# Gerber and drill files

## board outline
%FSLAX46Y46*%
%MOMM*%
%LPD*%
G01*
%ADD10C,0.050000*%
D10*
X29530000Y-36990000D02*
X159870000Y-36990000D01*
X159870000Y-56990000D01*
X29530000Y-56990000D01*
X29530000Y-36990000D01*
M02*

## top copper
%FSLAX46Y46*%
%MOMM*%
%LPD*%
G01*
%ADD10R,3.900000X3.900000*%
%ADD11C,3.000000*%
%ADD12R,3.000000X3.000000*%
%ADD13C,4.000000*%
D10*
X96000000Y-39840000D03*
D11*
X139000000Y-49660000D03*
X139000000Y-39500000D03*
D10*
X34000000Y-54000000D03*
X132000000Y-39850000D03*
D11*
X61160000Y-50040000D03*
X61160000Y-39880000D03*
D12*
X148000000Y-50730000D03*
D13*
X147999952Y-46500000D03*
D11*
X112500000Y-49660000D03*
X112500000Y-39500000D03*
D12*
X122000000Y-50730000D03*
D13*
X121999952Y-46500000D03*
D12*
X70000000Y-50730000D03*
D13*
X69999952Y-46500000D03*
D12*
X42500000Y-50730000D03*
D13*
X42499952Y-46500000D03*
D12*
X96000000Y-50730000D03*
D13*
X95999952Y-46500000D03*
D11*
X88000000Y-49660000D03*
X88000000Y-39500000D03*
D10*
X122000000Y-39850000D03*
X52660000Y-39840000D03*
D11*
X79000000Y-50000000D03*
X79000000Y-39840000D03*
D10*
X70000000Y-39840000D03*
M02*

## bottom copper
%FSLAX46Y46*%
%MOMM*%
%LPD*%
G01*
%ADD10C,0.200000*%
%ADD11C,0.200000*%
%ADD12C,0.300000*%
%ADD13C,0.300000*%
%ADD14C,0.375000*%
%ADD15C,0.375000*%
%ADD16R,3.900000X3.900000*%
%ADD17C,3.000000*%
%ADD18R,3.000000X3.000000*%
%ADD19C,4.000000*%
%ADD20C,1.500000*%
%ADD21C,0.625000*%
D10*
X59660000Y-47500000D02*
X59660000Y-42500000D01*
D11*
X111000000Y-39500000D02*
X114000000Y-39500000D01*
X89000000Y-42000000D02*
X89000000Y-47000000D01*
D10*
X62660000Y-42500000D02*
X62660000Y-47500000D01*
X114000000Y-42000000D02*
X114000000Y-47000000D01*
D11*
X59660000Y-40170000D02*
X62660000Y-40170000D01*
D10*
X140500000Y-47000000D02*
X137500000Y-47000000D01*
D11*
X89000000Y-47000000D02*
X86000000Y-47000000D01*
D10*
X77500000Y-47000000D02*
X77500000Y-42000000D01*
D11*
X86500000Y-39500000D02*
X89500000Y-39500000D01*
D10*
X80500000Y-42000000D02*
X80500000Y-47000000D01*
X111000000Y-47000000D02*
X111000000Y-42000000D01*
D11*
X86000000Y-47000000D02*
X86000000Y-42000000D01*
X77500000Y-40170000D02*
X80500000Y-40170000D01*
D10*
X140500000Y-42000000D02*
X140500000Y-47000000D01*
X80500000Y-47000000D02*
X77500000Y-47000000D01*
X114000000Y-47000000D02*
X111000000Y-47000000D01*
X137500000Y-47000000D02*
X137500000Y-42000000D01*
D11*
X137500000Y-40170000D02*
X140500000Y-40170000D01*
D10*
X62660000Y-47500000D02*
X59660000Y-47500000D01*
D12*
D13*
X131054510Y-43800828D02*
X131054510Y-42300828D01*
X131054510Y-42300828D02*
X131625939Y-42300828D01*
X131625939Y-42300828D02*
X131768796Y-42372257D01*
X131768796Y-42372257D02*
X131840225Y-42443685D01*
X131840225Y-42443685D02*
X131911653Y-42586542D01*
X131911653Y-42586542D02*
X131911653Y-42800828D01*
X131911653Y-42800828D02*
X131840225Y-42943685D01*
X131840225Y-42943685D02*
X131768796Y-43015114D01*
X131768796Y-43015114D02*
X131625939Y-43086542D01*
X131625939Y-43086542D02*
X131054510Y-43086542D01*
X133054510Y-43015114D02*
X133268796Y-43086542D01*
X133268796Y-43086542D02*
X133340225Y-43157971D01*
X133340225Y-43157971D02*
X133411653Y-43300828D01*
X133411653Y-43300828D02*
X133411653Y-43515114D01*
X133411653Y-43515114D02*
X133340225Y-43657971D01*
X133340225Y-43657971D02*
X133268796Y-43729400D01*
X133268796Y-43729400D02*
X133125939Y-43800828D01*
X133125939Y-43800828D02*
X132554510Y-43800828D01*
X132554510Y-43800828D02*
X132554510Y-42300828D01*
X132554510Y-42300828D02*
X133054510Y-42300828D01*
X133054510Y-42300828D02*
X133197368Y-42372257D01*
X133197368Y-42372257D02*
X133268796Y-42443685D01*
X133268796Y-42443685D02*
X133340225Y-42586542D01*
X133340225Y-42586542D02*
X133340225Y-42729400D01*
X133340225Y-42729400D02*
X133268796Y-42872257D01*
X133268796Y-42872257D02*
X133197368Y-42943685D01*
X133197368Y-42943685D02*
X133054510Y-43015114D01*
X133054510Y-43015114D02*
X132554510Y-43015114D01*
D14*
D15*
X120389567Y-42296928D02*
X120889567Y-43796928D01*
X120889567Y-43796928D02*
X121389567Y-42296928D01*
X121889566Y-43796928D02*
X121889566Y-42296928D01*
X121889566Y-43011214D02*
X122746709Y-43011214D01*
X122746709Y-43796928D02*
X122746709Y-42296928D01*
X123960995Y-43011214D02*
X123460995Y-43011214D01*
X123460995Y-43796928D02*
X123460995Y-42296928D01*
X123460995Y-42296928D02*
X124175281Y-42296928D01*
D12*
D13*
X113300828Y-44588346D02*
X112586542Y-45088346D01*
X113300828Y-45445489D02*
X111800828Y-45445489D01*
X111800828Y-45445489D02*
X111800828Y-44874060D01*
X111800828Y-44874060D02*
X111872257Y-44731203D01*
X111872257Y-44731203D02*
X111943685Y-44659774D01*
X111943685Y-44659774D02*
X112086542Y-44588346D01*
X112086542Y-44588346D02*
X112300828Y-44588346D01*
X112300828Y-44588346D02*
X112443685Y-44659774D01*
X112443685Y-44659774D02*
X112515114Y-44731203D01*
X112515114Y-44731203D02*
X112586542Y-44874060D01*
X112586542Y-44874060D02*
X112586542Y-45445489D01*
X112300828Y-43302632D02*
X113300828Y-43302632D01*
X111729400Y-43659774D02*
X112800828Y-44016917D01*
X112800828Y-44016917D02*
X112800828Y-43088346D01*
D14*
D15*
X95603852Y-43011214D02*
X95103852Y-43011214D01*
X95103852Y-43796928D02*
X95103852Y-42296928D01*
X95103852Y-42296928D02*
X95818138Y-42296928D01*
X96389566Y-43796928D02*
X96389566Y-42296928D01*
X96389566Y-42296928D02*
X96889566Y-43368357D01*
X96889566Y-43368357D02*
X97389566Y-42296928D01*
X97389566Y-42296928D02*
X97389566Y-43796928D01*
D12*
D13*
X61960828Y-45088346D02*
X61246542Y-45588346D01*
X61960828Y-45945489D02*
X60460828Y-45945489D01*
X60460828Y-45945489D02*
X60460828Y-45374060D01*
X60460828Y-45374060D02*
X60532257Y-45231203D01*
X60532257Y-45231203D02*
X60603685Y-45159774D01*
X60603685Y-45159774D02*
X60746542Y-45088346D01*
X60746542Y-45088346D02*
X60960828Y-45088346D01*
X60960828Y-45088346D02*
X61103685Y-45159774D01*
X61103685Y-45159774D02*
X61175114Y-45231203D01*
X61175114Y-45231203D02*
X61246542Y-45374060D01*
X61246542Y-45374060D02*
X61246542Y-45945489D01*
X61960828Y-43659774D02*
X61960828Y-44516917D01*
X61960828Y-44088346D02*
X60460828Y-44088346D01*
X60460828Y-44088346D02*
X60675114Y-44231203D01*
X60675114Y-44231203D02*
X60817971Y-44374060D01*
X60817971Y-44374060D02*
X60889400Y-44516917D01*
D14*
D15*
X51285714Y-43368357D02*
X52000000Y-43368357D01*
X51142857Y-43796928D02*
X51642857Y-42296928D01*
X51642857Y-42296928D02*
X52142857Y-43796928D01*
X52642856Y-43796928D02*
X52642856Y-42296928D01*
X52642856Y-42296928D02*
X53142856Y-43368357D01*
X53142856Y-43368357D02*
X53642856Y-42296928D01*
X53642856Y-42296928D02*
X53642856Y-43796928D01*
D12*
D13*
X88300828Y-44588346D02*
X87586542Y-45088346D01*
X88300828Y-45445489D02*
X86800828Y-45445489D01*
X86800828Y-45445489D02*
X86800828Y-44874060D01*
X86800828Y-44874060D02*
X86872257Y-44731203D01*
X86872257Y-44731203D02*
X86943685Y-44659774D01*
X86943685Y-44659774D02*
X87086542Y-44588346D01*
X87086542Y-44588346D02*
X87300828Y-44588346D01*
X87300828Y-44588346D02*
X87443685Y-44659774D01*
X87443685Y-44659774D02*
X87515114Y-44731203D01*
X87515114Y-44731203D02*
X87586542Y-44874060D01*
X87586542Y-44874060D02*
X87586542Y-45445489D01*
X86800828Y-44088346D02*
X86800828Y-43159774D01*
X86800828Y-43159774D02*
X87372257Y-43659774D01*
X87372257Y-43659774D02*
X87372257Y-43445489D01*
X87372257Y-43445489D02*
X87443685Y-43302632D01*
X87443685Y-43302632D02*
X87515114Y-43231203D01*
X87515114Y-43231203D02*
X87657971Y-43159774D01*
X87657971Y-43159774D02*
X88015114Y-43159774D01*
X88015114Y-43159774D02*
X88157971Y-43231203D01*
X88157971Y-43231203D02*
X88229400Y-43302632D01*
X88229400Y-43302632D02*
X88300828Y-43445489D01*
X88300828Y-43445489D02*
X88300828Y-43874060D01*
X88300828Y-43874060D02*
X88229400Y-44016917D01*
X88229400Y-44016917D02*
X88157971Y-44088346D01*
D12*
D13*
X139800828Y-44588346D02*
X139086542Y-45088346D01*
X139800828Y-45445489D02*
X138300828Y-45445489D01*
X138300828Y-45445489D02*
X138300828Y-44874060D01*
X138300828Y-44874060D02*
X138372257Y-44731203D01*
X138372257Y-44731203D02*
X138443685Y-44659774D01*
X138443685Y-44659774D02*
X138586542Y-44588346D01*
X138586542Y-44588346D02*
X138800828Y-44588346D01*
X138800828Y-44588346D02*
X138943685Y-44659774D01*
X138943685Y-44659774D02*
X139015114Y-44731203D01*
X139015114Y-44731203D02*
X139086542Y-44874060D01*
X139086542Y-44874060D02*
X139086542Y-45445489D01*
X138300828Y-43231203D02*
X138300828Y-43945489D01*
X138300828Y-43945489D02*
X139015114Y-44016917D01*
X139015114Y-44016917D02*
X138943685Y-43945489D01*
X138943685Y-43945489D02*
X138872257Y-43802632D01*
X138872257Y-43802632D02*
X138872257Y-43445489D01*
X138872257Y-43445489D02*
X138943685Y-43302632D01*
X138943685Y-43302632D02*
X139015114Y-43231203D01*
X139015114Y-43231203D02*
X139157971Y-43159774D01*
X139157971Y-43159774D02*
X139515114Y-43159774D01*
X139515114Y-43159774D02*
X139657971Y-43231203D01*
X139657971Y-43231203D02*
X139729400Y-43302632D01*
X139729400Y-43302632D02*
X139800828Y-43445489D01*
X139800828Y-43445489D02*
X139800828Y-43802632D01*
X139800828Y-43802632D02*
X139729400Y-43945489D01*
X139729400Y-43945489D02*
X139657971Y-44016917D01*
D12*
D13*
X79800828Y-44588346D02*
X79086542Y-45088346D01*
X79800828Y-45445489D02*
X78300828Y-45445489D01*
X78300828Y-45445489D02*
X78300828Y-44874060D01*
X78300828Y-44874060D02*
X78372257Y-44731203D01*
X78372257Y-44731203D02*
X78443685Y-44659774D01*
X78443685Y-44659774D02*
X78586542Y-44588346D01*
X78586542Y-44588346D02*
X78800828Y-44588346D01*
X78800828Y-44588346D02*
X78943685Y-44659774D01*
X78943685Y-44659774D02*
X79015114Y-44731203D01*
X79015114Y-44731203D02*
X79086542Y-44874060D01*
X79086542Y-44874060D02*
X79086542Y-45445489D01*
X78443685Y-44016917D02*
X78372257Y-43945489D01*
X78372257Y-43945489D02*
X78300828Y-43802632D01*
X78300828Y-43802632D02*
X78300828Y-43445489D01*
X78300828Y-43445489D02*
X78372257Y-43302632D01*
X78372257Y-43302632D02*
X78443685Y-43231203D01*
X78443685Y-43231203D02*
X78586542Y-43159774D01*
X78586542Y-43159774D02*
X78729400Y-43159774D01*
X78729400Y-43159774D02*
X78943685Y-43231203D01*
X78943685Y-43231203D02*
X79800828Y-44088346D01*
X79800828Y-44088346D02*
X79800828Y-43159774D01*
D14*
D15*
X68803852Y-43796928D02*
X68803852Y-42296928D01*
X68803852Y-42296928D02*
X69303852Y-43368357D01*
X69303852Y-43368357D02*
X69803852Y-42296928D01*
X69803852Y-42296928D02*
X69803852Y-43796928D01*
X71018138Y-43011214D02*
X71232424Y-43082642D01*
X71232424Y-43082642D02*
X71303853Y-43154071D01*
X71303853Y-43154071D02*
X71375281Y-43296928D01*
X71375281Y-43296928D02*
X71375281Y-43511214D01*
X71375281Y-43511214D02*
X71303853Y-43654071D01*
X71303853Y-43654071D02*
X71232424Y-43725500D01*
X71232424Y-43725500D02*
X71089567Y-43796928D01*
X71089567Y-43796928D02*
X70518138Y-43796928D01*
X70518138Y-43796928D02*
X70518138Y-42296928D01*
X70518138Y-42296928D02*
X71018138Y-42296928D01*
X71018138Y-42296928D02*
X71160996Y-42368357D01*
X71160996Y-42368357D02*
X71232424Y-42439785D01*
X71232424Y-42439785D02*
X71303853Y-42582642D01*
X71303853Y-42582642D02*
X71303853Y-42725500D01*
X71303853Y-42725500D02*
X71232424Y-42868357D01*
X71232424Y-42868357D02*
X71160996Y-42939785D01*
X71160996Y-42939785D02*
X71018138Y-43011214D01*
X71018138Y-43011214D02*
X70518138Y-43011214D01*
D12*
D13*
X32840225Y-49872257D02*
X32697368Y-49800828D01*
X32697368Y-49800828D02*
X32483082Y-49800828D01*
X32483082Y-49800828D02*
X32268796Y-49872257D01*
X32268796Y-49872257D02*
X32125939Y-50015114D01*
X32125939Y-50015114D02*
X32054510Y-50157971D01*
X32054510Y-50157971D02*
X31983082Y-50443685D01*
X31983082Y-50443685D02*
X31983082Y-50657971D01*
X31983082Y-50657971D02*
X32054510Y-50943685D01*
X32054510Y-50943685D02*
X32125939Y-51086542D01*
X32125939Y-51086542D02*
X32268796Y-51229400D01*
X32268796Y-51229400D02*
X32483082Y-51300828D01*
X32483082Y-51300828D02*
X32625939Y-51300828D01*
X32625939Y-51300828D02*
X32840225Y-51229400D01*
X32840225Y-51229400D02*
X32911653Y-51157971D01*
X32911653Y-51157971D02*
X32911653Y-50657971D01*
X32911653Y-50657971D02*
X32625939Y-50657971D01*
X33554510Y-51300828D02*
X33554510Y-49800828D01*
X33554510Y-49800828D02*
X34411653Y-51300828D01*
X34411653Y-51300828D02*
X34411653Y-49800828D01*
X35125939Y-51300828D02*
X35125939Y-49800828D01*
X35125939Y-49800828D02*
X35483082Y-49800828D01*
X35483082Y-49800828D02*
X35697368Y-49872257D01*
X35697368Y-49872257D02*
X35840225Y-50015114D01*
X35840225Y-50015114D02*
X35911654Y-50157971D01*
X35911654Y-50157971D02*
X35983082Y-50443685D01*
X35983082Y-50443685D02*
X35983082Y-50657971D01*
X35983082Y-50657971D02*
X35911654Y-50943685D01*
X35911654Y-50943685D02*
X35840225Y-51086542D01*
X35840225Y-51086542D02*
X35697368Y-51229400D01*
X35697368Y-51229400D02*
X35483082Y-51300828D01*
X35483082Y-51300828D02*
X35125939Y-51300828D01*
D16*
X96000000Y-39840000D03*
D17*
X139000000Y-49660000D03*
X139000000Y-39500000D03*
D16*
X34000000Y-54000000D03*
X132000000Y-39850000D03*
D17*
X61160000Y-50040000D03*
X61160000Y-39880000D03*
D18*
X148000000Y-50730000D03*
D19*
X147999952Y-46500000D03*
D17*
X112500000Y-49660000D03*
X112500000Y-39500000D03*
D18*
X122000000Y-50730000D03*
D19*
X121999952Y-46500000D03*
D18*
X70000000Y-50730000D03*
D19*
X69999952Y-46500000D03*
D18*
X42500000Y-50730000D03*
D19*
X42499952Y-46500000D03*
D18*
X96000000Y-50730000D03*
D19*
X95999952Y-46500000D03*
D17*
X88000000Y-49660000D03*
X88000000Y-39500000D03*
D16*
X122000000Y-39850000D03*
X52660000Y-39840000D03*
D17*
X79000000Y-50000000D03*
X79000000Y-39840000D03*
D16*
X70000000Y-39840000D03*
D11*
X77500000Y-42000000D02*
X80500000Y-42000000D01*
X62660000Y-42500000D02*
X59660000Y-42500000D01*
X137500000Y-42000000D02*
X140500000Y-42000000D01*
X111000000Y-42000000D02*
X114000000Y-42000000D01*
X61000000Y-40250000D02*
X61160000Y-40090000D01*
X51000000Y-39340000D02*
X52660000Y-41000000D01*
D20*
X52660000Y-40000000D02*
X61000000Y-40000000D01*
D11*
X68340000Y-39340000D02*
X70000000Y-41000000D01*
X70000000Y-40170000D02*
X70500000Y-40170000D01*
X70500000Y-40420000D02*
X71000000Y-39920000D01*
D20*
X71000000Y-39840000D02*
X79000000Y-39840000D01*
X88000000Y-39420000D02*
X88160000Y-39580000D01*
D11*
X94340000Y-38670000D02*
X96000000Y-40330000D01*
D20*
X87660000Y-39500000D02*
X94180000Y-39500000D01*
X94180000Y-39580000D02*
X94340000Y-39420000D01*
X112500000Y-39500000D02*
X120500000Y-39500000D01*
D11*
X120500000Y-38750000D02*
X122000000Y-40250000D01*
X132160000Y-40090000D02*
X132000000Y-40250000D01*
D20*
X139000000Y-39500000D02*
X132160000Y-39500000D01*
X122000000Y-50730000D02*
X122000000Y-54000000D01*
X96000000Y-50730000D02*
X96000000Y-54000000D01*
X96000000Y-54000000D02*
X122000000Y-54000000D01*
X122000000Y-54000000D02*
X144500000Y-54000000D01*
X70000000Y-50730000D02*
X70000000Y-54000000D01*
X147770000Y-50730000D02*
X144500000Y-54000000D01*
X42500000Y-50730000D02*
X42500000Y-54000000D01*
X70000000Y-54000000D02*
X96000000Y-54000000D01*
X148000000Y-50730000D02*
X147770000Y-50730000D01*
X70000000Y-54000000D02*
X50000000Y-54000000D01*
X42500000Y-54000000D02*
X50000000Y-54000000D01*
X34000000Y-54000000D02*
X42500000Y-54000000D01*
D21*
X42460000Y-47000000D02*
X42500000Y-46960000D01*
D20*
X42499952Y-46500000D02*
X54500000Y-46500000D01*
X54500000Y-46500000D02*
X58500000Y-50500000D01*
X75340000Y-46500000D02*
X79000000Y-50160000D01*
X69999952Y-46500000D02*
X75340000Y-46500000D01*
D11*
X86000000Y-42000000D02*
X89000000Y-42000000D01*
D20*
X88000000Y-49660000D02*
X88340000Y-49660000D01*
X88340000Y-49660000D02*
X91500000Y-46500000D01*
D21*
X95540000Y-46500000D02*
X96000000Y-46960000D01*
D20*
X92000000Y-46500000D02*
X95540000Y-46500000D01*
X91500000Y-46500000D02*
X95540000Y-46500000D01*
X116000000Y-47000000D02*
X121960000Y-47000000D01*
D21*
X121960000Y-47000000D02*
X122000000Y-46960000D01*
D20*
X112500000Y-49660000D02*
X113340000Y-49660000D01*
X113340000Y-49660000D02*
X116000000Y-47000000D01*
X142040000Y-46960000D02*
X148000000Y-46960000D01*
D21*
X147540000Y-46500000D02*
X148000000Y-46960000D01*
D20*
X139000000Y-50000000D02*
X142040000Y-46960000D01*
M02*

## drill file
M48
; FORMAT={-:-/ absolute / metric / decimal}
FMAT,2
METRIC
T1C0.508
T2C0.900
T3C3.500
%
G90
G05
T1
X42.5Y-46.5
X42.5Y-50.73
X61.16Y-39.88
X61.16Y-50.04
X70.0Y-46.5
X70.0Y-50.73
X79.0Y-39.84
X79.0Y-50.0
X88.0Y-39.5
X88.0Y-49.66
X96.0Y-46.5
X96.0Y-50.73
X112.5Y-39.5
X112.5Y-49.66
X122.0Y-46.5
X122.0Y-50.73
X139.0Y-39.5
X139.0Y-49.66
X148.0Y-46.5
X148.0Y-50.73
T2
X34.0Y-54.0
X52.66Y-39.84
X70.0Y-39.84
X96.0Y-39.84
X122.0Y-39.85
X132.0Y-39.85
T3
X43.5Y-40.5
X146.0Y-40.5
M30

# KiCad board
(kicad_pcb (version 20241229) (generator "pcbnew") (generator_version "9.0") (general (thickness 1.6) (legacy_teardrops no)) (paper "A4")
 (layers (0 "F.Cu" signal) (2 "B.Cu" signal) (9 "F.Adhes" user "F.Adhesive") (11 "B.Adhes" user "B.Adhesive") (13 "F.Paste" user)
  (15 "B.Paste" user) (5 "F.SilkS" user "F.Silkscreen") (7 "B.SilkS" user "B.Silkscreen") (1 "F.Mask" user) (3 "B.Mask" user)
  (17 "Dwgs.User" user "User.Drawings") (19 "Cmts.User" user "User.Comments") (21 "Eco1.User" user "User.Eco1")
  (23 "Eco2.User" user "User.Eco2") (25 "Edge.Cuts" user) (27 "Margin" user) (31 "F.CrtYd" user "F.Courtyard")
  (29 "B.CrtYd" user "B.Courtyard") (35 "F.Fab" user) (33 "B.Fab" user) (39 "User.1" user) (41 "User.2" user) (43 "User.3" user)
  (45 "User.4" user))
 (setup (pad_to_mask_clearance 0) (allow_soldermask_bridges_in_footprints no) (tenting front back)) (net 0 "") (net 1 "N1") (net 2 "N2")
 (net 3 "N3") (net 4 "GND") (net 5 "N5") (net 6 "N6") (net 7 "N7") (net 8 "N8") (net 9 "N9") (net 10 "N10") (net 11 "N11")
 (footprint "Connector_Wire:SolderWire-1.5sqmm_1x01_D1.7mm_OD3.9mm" (layer "F.Cu") (at 96 39.5 90)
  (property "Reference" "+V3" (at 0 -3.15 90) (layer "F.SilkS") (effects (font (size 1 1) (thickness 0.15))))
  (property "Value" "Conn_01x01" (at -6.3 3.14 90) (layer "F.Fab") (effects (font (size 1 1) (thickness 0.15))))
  (pad "1" thru_hole rect (at -0.34 0 90) (size 3.9 3.9) (drill 0.9) (layers "*.Cu" "*.Mask") (remove_unused_layers no) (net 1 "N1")))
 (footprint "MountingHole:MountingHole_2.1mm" (layer "F.Cu") (at 43.5 40.5)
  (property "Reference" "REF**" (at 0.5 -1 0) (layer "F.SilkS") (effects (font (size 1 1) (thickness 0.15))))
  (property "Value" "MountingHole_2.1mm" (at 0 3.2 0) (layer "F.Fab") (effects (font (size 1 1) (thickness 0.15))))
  (pad "" np_thru_hole circle (at 0 0) (size 2.1 2.1) (drill 3.5) (layers "*.Cu" "*.Mask")))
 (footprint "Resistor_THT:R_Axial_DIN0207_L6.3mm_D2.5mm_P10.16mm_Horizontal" (layer "F.Cu") (at 139 49.66 90)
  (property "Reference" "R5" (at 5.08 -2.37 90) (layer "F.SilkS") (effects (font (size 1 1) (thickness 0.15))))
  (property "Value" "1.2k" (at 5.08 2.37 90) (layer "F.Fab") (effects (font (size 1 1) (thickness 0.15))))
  (pad "1" thru_hole circle (at 0 0 90) (size 3 3) (drill 0.508) (layers "*.Cu" "*.Mask") (remove_unused_layers no) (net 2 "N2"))
  (pad "2" thru_hole circle (at 10.16 0 90) (size 3 3) (drill 0.508) (layers "*.Cu" "*.Mask") (remove_unused_layers no) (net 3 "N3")))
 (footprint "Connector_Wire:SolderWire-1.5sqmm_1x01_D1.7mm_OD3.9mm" (layer "F.Cu") (at 34 54)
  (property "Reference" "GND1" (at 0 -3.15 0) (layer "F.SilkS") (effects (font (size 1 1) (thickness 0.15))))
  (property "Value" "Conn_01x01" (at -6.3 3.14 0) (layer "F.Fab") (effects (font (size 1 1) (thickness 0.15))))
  (pad "1" thru_hole rect (at 0 0) (size 3.9 3.9) (drill 0.9) (layers "*.Cu" "*.Mask") (remove_unused_layers no) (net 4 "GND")))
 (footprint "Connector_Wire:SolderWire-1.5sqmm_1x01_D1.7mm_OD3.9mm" (layer "F.Cu") (at 132 39.5 90)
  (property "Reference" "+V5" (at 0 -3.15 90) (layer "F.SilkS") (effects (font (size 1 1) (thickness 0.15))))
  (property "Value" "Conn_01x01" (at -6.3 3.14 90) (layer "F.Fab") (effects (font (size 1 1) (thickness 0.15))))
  (pad "1" thru_hole rect (at -0.35 0 90) (size 3.9 3.9) (drill 0.9) (layers "*.Cu" "*.Mask") (remove_unused_layers no) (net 3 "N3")))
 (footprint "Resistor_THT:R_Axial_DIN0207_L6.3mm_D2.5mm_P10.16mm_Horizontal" (layer "F.Cu") (at 61.16 50.04 90)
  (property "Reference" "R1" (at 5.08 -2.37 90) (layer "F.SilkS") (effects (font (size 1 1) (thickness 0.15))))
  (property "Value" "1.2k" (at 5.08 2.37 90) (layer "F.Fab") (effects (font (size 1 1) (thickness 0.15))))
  (pad "1" thru_hole circle (at 0 0 90) (size 3 3) (drill 0.508) (layers "*.Cu" "*.Mask") (remove_unused_layers no) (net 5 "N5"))
  (pad "2" thru_hole circle (at 10.16 0 90) (size 3 3) (drill 0.508) (layers "*.Cu" "*.Mask") (remove_unused_layers no) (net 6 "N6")))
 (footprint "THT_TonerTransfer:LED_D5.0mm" (layer "F.Cu") (at 148 49.5 90)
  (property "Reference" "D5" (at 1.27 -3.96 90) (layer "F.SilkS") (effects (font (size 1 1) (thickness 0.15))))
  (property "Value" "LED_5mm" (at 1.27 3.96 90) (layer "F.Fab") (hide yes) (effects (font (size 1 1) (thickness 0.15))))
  (pad "1" thru_hole rect (at -1.23 0 90) (size 3 3) (drill 0.508) (layers "*.Cu" "*.Mask") (remove_unused_layers no) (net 4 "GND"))
  (pad "2" thru_hole circle (at 3 -0.000048 90) (size 4 4) (drill 0.508) (layers "*.Cu" "*.Mask") (remove_unused_layers no) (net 2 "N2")))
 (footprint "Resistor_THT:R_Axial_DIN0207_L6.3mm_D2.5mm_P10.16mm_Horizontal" (layer "F.Cu") (at 112.5 49.66 90)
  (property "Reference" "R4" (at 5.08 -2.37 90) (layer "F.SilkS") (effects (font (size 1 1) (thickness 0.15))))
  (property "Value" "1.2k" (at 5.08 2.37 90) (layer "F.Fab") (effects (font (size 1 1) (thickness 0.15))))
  (pad "1" thru_hole circle (at 0 0 90) (size 3 3) (drill 0.508) (layers "*.Cu" "*.Mask") (remove_unused_layers no) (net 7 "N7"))
  (pad "2" thru_hole circle (at 10.16 0 90) (size 3 3) (drill 0.508) (layers "*.Cu" "*.Mask") (remove_unused_layers no) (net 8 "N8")))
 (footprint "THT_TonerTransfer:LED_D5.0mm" (layer "F.Cu") (at 122 49.5 90)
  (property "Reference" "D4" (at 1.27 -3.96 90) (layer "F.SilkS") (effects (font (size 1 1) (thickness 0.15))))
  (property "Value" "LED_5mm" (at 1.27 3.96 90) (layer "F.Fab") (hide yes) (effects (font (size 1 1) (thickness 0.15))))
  (pad "1" thru_hole rect (at -1.23 0 90) (size 3 3) (drill 0.508) (layers "*.Cu" "*.Mask") (remove_unused_layers no) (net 4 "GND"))
  (pad "2" thru_hole circle (at 3 -0.000048 90) (size 4 4) (drill 0.508) (layers "*.Cu" "*.Mask") (remove_unused_layers no) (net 7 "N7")))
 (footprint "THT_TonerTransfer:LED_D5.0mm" (layer "F.Cu") (at 70 49.5 90)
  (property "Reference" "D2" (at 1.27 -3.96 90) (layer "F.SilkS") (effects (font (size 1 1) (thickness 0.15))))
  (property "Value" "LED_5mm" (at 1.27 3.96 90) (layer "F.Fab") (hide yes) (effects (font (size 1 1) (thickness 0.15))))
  (pad "1" thru_hole rect (at -1.23 0 90) (size 3 3) (drill 0.508) (layers "*.Cu" "*.Mask") (remove_unused_layers no) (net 4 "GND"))
  (pad "2" thru_hole circle (at 3 -0.000048 90) (size 4 4) (drill 0.508) (layers "*.Cu" "*.Mask") (remove_unused_layers no) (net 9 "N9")))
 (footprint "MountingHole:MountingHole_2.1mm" (layer "F.Cu") (at 146 40.5)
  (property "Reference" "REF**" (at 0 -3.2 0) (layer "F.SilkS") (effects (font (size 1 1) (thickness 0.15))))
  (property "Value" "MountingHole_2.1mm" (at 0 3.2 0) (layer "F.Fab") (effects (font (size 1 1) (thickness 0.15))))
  (pad "" np_thru_hole circle (at 0 0) (size 2.1 2.1) (drill 3.5) (layers "*.Cu" "*.Mask")))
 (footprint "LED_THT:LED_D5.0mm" (layer "F.Cu") (at 42.5 49.5 90)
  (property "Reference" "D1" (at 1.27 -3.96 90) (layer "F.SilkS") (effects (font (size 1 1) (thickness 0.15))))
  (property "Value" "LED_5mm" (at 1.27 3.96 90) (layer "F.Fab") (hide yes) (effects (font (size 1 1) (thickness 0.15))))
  (pad "1" thru_hole rect (at -1.23 0 90) (size 3 3) (drill 0.508) (layers "*.Cu" "*.Mask") (remove_unused_layers no) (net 4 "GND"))
  (pad "2" thru_hole circle (at 3 -0.000048 90) (size 4 4) (drill 0.508) (layers "*.Cu" "*.Mask") (remove_unused_layers no) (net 5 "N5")))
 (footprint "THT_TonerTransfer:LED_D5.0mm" (layer "F.Cu") (at 96 49.5 90)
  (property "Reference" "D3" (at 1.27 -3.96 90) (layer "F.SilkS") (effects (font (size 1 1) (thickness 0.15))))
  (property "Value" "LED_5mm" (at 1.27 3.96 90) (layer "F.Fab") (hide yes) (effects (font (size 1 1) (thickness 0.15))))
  (pad "1" thru_hole rect (at -1.23 0 90) (size 3 3) (drill 0.508) (layers "*.Cu" "*.Mask") (remove_unused_layers no) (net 4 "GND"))
  (pad "2" thru_hole circle (at 3 -0.000048 90) (size 4 4) (drill 0.508) (layers "*.Cu" "*.Mask") (remove_unused_layers no) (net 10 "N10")))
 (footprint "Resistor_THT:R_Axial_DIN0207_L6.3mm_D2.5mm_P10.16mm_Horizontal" (layer "F.Cu") (at 88 49.66 90)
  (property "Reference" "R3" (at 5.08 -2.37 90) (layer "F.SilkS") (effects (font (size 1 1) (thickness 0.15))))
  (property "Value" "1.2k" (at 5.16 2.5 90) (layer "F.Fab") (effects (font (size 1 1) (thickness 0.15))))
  (pad "1" thru_hole circle (at 0 0 90) (size 3 3) (drill 0.508) (layers "*.Cu" "*.Mask") (remove_unused_layers no) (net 10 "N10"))
  (pad "2" thru_hole circle (at 10.16 0 90) (size 3 3) (drill 0.508) (layers "*.Cu" "*.Mask") (remove_unused_layers no) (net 1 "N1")))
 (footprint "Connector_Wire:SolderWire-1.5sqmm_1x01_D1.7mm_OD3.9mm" (layer "F.Cu") (at 122 39.5 90)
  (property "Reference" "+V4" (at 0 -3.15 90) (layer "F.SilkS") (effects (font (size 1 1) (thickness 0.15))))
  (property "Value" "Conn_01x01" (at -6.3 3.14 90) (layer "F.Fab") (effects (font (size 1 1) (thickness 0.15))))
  (pad "1" thru_hole rect (at -0.35 0 90) (size 3.9 3.9) (drill 0.9) (layers "*.Cu" "*.Mask") (remove_unused_layers no) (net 8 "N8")))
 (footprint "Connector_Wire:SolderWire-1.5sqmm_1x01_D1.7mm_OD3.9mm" (layer "F.Cu") (at 52.66 40 90)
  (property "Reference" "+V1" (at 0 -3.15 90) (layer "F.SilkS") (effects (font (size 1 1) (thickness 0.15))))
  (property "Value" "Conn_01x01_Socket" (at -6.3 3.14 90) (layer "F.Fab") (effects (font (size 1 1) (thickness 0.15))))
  (pad "1" thru_hole rect (at 0.16 0 90) (size 3.9 3.9) (drill 0.9) (layers "*.Cu" "*.Mask") (remove_unused_layers no) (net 6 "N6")))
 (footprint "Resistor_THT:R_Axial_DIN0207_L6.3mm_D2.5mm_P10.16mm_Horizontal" (layer "F.Cu") (at 79 50 90)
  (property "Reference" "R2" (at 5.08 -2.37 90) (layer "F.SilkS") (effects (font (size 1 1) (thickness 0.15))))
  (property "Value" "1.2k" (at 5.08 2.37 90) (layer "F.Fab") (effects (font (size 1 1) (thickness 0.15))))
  (pad "1" thru_hole circle (at 0 0 90) (size 3 3) (drill 0.508) (layers "*.Cu" "*.Mask") (remove_unused_layers no) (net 9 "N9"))
  (pad "2" thru_hole circle (at 10.16 0 90) (size 3 3) (drill 0.508) (layers "*.Cu" "*.Mask") (remove_unused_layers no) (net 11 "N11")))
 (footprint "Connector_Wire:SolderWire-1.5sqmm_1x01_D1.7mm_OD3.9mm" (layer "F.Cu") (at 70 39.84 90)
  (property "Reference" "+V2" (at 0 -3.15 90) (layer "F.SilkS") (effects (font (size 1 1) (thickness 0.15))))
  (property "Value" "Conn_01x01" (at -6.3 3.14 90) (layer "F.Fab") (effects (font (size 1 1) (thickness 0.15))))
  (pad "1" thru_hole rect (at 0 0 90) (size 3.9 3.9) (drill 0.9) (layers "*.Cu" "*.Mask") (remove_unused_layers no) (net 11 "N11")))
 (gr_line (start 59.66 47.5) (end 59.66 42.5) (stroke (width 0.2) (type default)) (layer "B.Cu"))
 (gr_line (start 111 39.5) (end 114 39.5) (stroke (width 0.2) (type default)) (layer "B.Cu") (net 8))
 (gr_line (start 89 42) (end 89 47) (stroke (width 0.2) (type default)) (layer "B.Cu") (net 10))
 (gr_line (start 62.66 42.5) (end 62.66 47.5) (stroke (width 0.2) (type default)) (layer "B.Cu"))
 (gr_line (start 114 42) (end 114 47) (stroke (width 0.2) (type default)) (layer "B.Cu"))
 (gr_line (start 59.66 40.17) (end 62.66 40.17) (stroke (width 0.2) (type default)) (layer "B.Cu") (net 6))
 (gr_line (start 140.5 47) (end 137.5 47) (stroke (width 0.2) (type default)) (layer "B.Cu"))
 (gr_line (start 89 47) (end 86 47) (stroke (width 0.2) (type default)) (layer "B.Cu") (net 10))
 (gr_line (start 77.5 47) (end 77.5 42) (stroke (width 0.2) (type default)) (layer "B.Cu"))
 (gr_line (start 86.5 39.5) (end 89.5 39.5) (stroke (width 0.2) (type default)) (layer "B.Cu") (net 1))
 (gr_line (start 80.5 42) (end 80.5 47) (stroke (width 0.2) (type default)) (layer "B.Cu"))
 (gr_line (start 111 47) (end 111 42) (stroke (width 0.2) (type default)) (layer "B.Cu"))
 (gr_line (start 86 47) (end 86 42) (stroke (width 0.2) (type default)) (layer "B.Cu") (net 10))
 (gr_line (start 77.5 40.17) (end 80.5 40.17) (stroke (width 0.2) (type default)) (layer "B.Cu") (net 11))
 (gr_line (start 140.5 42) (end 140.5 47) (stroke (width 0.2) (type default)) (layer "B.Cu"))
 (gr_line (start 80.5 47) (end 77.5 47) (stroke (width 0.2) (type default)) (layer "B.Cu"))
 (gr_line (start 114 47) (end 111 47) (stroke (width 0.2) (type default)) (layer "B.Cu"))
 (gr_line (start 137.5 47) (end 137.5 42) (stroke (width 0.2) (type default)) (layer "B.Cu"))
 (gr_line (start 137.5 40.17) (end 140.5 40.17) (stroke (width 0.2) (type default)) (layer "B.Cu") (net 3))
 (gr_line (start 62.66 47.5) (end 59.66 47.5) (stroke (width 0.2) (type default)) (layer "B.Cu"))
 (gr_rect (start 29.53 36.99) (end 159.87 56.99) (stroke (width 0.05) (type solid)) (fill no) (locked yes) (layer "Edge.Cuts"))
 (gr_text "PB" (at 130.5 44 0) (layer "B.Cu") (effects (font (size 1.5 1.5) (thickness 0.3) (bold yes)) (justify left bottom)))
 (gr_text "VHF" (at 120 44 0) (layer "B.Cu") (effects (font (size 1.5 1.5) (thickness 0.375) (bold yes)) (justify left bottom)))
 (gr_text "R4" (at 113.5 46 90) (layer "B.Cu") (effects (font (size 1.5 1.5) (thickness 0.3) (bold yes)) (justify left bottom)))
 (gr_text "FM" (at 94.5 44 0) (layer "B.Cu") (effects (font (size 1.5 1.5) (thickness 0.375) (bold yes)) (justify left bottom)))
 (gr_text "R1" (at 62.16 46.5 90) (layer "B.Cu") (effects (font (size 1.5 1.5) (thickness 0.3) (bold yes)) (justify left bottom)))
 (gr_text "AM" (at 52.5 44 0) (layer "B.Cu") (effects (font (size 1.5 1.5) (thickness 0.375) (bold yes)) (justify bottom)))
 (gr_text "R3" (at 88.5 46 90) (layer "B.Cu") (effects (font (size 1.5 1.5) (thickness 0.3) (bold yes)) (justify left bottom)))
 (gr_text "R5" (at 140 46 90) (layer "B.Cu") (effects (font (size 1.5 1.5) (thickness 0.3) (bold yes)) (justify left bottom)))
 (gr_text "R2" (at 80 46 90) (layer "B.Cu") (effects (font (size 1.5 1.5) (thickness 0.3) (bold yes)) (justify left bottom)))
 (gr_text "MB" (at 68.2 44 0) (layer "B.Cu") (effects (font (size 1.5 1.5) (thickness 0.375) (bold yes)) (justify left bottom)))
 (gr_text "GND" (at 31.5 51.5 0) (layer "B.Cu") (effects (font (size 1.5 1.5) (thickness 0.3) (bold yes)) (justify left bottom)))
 (segment (start 77.5 42) (end 80.5 42) (width 0.2) (layer "B.Cu") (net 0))
 (segment (start 62.66 42.5) (end 59.66 42.5) (width 0.2) (layer "B.Cu") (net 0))
 (segment (start 137.5 42) (end 140.5 42) (width 0.2) (layer "B.Cu") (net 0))
 (segment (start 111 42) (end 114 42) (width 0.2) (layer "B.Cu") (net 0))
 (segment (start 61 40.25) (end 61.16 40.09) (width 0.2) (layer "B.Cu") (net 6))
 (segment (start 51 39.34) (end 52.66 41) (width 0.2) (layer "B.Cu") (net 6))
 (segment (start 52.66 40) (end 61 40) (width 1.5) (layer "B.Cu") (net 6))
 (segment (start 68.34 39.34) (end 70 41) (width 0.2) (layer "B.Cu") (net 11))
 (segment (start 70 40.17) (end 70.5 40.17) (width 0.2) (layer "B.Cu") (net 11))
 (segment (start 70.5 40.42) (end 71 39.92) (width 0.2) (layer "B.Cu") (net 11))
 (segment (start 71 39.84) (end 79 39.84) (width 1.5) (layer "B.Cu") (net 11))
 (segment (start 88 39.42) (end 88.16 39.58) (width 1.5) (layer "B.Cu") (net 1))
 (segment (start 94.34 38.67) (end 96 40.33) (width 0.2) (layer "B.Cu") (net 1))
 (segment (start 87.66 39.5) (end 94.18 39.5) (width 1.5) (layer "B.Cu") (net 1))
 (segment (start 94.18 39.58) (end 94.34 39.42) (width 1.5) (layer "B.Cu") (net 1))
 (segment (start 112.5 39.5) (end 120.5 39.5) (width 1.5) (layer "B.Cu") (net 8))
 (segment (start 120.5 38.75) (end 122 40.25) (width 0.2) (layer "B.Cu") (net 8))
 (segment (start 132.16 40.09) (end 132 40.25) (width 0.2) (layer "B.Cu") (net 3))
 (segment (start 139 39.5) (end 132.16 39.5) (width 1.5) (layer "B.Cu") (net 3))
 (segment (start 122 50.73) (end 122 54) (width 1.5) (layer "B.Cu") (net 4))
 (segment (start 96 50.73) (end 96 54) (width 1.5) (layer "B.Cu") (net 4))
 (segment (start 96 54) (end 122 54) (width 1.5) (layer "B.Cu") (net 4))
 (segment (start 122 54) (end 144.5 54) (width 1.5) (layer "B.Cu") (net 4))
 (segment (start 70 50.73) (end 70 54) (width 1.5) (layer "B.Cu") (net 4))
 (segment (start 147.77 50.73) (end 144.5 54) (width 1.5) (layer "B.Cu") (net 4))
 (segment (start 42.5 50.73) (end 42.5 54) (width 1.5) (layer "B.Cu") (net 4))
 (segment (start 70 54) (end 96 54) (width 1.5) (layer "B.Cu") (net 4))
 (segment (start 148 50.73) (end 147.77 50.73) (width 1.5) (layer "B.Cu") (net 4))
 (segment (start 70 54) (end 50 54) (width 1.5) (layer "B.Cu") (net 4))
 (segment (start 42.5 54) (end 50 54) (width 1.5) (layer "B.Cu") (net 4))
 (segment (start 34 54) (end 42.5 54) (width 1.5) (layer "B.Cu") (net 4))
 (segment (start 42.46 47) (end 42.5 46.96) (width 0.625) (layer "B.Cu") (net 5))
 (segment (start 42.499952 46.5) (end 54.5 46.5) (width 1.5) (layer "B.Cu") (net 5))
 (segment (start 54.5 46.5) (end 58.5 50.5) (width 1.5) (layer "B.Cu") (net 5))
 (segment (start 75.34 46.5) (end 79 50.16) (width 1.5) (layer "B.Cu") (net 9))
 (segment (start 69.999952 46.5) (end 75.34 46.5) (width 1.5) (layer "B.Cu") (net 9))
 (segment (start 86 42) (end 89 42) (width 0.2) (layer "B.Cu") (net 10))
 (segment (start 88 49.66) (end 88.34 49.66) (width 1.5) (layer "B.Cu") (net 10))
 (segment (start 88.34 49.66) (end 91.5 46.5) (width 1.5) (layer "B.Cu") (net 10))
 (segment (start 95.54 46.5) (end 96 46.96) (width 0.625) (layer "B.Cu") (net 10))
 (segment (start 92 46.5) (end 95.54 46.5) (width 1.5) (layer "B.Cu") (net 10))
 (segment (start 91.5 46.5) (end 95.54 46.5) (width 1.5) (layer "B.Cu") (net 10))
 (segment (start 116 47) (end 121.96 47) (width 1.5) (layer "B.Cu") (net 7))
 (segment (start 121.96 47) (end 122 46.96) (width 0.625) (layer "B.Cu") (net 7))
 (segment (start 112.5 49.66) (end 113.34 49.66) (width 1.5) (layer "B.Cu") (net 7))
 (segment (start 113.34 49.66) (end 116 47) (width 1.5) (layer "B.Cu") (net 7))
 (segment (start 142.04 46.96) (end 148 46.96) (width 1.5) (layer "B.Cu") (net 2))
 (segment (start 147.54 46.5) (end 148 46.96) (width 0.625) (layer "B.Cu") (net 2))
 (segment (start 139 50) (end 142.04 46.96) (width 1.5) (layer "B.Cu") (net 2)))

